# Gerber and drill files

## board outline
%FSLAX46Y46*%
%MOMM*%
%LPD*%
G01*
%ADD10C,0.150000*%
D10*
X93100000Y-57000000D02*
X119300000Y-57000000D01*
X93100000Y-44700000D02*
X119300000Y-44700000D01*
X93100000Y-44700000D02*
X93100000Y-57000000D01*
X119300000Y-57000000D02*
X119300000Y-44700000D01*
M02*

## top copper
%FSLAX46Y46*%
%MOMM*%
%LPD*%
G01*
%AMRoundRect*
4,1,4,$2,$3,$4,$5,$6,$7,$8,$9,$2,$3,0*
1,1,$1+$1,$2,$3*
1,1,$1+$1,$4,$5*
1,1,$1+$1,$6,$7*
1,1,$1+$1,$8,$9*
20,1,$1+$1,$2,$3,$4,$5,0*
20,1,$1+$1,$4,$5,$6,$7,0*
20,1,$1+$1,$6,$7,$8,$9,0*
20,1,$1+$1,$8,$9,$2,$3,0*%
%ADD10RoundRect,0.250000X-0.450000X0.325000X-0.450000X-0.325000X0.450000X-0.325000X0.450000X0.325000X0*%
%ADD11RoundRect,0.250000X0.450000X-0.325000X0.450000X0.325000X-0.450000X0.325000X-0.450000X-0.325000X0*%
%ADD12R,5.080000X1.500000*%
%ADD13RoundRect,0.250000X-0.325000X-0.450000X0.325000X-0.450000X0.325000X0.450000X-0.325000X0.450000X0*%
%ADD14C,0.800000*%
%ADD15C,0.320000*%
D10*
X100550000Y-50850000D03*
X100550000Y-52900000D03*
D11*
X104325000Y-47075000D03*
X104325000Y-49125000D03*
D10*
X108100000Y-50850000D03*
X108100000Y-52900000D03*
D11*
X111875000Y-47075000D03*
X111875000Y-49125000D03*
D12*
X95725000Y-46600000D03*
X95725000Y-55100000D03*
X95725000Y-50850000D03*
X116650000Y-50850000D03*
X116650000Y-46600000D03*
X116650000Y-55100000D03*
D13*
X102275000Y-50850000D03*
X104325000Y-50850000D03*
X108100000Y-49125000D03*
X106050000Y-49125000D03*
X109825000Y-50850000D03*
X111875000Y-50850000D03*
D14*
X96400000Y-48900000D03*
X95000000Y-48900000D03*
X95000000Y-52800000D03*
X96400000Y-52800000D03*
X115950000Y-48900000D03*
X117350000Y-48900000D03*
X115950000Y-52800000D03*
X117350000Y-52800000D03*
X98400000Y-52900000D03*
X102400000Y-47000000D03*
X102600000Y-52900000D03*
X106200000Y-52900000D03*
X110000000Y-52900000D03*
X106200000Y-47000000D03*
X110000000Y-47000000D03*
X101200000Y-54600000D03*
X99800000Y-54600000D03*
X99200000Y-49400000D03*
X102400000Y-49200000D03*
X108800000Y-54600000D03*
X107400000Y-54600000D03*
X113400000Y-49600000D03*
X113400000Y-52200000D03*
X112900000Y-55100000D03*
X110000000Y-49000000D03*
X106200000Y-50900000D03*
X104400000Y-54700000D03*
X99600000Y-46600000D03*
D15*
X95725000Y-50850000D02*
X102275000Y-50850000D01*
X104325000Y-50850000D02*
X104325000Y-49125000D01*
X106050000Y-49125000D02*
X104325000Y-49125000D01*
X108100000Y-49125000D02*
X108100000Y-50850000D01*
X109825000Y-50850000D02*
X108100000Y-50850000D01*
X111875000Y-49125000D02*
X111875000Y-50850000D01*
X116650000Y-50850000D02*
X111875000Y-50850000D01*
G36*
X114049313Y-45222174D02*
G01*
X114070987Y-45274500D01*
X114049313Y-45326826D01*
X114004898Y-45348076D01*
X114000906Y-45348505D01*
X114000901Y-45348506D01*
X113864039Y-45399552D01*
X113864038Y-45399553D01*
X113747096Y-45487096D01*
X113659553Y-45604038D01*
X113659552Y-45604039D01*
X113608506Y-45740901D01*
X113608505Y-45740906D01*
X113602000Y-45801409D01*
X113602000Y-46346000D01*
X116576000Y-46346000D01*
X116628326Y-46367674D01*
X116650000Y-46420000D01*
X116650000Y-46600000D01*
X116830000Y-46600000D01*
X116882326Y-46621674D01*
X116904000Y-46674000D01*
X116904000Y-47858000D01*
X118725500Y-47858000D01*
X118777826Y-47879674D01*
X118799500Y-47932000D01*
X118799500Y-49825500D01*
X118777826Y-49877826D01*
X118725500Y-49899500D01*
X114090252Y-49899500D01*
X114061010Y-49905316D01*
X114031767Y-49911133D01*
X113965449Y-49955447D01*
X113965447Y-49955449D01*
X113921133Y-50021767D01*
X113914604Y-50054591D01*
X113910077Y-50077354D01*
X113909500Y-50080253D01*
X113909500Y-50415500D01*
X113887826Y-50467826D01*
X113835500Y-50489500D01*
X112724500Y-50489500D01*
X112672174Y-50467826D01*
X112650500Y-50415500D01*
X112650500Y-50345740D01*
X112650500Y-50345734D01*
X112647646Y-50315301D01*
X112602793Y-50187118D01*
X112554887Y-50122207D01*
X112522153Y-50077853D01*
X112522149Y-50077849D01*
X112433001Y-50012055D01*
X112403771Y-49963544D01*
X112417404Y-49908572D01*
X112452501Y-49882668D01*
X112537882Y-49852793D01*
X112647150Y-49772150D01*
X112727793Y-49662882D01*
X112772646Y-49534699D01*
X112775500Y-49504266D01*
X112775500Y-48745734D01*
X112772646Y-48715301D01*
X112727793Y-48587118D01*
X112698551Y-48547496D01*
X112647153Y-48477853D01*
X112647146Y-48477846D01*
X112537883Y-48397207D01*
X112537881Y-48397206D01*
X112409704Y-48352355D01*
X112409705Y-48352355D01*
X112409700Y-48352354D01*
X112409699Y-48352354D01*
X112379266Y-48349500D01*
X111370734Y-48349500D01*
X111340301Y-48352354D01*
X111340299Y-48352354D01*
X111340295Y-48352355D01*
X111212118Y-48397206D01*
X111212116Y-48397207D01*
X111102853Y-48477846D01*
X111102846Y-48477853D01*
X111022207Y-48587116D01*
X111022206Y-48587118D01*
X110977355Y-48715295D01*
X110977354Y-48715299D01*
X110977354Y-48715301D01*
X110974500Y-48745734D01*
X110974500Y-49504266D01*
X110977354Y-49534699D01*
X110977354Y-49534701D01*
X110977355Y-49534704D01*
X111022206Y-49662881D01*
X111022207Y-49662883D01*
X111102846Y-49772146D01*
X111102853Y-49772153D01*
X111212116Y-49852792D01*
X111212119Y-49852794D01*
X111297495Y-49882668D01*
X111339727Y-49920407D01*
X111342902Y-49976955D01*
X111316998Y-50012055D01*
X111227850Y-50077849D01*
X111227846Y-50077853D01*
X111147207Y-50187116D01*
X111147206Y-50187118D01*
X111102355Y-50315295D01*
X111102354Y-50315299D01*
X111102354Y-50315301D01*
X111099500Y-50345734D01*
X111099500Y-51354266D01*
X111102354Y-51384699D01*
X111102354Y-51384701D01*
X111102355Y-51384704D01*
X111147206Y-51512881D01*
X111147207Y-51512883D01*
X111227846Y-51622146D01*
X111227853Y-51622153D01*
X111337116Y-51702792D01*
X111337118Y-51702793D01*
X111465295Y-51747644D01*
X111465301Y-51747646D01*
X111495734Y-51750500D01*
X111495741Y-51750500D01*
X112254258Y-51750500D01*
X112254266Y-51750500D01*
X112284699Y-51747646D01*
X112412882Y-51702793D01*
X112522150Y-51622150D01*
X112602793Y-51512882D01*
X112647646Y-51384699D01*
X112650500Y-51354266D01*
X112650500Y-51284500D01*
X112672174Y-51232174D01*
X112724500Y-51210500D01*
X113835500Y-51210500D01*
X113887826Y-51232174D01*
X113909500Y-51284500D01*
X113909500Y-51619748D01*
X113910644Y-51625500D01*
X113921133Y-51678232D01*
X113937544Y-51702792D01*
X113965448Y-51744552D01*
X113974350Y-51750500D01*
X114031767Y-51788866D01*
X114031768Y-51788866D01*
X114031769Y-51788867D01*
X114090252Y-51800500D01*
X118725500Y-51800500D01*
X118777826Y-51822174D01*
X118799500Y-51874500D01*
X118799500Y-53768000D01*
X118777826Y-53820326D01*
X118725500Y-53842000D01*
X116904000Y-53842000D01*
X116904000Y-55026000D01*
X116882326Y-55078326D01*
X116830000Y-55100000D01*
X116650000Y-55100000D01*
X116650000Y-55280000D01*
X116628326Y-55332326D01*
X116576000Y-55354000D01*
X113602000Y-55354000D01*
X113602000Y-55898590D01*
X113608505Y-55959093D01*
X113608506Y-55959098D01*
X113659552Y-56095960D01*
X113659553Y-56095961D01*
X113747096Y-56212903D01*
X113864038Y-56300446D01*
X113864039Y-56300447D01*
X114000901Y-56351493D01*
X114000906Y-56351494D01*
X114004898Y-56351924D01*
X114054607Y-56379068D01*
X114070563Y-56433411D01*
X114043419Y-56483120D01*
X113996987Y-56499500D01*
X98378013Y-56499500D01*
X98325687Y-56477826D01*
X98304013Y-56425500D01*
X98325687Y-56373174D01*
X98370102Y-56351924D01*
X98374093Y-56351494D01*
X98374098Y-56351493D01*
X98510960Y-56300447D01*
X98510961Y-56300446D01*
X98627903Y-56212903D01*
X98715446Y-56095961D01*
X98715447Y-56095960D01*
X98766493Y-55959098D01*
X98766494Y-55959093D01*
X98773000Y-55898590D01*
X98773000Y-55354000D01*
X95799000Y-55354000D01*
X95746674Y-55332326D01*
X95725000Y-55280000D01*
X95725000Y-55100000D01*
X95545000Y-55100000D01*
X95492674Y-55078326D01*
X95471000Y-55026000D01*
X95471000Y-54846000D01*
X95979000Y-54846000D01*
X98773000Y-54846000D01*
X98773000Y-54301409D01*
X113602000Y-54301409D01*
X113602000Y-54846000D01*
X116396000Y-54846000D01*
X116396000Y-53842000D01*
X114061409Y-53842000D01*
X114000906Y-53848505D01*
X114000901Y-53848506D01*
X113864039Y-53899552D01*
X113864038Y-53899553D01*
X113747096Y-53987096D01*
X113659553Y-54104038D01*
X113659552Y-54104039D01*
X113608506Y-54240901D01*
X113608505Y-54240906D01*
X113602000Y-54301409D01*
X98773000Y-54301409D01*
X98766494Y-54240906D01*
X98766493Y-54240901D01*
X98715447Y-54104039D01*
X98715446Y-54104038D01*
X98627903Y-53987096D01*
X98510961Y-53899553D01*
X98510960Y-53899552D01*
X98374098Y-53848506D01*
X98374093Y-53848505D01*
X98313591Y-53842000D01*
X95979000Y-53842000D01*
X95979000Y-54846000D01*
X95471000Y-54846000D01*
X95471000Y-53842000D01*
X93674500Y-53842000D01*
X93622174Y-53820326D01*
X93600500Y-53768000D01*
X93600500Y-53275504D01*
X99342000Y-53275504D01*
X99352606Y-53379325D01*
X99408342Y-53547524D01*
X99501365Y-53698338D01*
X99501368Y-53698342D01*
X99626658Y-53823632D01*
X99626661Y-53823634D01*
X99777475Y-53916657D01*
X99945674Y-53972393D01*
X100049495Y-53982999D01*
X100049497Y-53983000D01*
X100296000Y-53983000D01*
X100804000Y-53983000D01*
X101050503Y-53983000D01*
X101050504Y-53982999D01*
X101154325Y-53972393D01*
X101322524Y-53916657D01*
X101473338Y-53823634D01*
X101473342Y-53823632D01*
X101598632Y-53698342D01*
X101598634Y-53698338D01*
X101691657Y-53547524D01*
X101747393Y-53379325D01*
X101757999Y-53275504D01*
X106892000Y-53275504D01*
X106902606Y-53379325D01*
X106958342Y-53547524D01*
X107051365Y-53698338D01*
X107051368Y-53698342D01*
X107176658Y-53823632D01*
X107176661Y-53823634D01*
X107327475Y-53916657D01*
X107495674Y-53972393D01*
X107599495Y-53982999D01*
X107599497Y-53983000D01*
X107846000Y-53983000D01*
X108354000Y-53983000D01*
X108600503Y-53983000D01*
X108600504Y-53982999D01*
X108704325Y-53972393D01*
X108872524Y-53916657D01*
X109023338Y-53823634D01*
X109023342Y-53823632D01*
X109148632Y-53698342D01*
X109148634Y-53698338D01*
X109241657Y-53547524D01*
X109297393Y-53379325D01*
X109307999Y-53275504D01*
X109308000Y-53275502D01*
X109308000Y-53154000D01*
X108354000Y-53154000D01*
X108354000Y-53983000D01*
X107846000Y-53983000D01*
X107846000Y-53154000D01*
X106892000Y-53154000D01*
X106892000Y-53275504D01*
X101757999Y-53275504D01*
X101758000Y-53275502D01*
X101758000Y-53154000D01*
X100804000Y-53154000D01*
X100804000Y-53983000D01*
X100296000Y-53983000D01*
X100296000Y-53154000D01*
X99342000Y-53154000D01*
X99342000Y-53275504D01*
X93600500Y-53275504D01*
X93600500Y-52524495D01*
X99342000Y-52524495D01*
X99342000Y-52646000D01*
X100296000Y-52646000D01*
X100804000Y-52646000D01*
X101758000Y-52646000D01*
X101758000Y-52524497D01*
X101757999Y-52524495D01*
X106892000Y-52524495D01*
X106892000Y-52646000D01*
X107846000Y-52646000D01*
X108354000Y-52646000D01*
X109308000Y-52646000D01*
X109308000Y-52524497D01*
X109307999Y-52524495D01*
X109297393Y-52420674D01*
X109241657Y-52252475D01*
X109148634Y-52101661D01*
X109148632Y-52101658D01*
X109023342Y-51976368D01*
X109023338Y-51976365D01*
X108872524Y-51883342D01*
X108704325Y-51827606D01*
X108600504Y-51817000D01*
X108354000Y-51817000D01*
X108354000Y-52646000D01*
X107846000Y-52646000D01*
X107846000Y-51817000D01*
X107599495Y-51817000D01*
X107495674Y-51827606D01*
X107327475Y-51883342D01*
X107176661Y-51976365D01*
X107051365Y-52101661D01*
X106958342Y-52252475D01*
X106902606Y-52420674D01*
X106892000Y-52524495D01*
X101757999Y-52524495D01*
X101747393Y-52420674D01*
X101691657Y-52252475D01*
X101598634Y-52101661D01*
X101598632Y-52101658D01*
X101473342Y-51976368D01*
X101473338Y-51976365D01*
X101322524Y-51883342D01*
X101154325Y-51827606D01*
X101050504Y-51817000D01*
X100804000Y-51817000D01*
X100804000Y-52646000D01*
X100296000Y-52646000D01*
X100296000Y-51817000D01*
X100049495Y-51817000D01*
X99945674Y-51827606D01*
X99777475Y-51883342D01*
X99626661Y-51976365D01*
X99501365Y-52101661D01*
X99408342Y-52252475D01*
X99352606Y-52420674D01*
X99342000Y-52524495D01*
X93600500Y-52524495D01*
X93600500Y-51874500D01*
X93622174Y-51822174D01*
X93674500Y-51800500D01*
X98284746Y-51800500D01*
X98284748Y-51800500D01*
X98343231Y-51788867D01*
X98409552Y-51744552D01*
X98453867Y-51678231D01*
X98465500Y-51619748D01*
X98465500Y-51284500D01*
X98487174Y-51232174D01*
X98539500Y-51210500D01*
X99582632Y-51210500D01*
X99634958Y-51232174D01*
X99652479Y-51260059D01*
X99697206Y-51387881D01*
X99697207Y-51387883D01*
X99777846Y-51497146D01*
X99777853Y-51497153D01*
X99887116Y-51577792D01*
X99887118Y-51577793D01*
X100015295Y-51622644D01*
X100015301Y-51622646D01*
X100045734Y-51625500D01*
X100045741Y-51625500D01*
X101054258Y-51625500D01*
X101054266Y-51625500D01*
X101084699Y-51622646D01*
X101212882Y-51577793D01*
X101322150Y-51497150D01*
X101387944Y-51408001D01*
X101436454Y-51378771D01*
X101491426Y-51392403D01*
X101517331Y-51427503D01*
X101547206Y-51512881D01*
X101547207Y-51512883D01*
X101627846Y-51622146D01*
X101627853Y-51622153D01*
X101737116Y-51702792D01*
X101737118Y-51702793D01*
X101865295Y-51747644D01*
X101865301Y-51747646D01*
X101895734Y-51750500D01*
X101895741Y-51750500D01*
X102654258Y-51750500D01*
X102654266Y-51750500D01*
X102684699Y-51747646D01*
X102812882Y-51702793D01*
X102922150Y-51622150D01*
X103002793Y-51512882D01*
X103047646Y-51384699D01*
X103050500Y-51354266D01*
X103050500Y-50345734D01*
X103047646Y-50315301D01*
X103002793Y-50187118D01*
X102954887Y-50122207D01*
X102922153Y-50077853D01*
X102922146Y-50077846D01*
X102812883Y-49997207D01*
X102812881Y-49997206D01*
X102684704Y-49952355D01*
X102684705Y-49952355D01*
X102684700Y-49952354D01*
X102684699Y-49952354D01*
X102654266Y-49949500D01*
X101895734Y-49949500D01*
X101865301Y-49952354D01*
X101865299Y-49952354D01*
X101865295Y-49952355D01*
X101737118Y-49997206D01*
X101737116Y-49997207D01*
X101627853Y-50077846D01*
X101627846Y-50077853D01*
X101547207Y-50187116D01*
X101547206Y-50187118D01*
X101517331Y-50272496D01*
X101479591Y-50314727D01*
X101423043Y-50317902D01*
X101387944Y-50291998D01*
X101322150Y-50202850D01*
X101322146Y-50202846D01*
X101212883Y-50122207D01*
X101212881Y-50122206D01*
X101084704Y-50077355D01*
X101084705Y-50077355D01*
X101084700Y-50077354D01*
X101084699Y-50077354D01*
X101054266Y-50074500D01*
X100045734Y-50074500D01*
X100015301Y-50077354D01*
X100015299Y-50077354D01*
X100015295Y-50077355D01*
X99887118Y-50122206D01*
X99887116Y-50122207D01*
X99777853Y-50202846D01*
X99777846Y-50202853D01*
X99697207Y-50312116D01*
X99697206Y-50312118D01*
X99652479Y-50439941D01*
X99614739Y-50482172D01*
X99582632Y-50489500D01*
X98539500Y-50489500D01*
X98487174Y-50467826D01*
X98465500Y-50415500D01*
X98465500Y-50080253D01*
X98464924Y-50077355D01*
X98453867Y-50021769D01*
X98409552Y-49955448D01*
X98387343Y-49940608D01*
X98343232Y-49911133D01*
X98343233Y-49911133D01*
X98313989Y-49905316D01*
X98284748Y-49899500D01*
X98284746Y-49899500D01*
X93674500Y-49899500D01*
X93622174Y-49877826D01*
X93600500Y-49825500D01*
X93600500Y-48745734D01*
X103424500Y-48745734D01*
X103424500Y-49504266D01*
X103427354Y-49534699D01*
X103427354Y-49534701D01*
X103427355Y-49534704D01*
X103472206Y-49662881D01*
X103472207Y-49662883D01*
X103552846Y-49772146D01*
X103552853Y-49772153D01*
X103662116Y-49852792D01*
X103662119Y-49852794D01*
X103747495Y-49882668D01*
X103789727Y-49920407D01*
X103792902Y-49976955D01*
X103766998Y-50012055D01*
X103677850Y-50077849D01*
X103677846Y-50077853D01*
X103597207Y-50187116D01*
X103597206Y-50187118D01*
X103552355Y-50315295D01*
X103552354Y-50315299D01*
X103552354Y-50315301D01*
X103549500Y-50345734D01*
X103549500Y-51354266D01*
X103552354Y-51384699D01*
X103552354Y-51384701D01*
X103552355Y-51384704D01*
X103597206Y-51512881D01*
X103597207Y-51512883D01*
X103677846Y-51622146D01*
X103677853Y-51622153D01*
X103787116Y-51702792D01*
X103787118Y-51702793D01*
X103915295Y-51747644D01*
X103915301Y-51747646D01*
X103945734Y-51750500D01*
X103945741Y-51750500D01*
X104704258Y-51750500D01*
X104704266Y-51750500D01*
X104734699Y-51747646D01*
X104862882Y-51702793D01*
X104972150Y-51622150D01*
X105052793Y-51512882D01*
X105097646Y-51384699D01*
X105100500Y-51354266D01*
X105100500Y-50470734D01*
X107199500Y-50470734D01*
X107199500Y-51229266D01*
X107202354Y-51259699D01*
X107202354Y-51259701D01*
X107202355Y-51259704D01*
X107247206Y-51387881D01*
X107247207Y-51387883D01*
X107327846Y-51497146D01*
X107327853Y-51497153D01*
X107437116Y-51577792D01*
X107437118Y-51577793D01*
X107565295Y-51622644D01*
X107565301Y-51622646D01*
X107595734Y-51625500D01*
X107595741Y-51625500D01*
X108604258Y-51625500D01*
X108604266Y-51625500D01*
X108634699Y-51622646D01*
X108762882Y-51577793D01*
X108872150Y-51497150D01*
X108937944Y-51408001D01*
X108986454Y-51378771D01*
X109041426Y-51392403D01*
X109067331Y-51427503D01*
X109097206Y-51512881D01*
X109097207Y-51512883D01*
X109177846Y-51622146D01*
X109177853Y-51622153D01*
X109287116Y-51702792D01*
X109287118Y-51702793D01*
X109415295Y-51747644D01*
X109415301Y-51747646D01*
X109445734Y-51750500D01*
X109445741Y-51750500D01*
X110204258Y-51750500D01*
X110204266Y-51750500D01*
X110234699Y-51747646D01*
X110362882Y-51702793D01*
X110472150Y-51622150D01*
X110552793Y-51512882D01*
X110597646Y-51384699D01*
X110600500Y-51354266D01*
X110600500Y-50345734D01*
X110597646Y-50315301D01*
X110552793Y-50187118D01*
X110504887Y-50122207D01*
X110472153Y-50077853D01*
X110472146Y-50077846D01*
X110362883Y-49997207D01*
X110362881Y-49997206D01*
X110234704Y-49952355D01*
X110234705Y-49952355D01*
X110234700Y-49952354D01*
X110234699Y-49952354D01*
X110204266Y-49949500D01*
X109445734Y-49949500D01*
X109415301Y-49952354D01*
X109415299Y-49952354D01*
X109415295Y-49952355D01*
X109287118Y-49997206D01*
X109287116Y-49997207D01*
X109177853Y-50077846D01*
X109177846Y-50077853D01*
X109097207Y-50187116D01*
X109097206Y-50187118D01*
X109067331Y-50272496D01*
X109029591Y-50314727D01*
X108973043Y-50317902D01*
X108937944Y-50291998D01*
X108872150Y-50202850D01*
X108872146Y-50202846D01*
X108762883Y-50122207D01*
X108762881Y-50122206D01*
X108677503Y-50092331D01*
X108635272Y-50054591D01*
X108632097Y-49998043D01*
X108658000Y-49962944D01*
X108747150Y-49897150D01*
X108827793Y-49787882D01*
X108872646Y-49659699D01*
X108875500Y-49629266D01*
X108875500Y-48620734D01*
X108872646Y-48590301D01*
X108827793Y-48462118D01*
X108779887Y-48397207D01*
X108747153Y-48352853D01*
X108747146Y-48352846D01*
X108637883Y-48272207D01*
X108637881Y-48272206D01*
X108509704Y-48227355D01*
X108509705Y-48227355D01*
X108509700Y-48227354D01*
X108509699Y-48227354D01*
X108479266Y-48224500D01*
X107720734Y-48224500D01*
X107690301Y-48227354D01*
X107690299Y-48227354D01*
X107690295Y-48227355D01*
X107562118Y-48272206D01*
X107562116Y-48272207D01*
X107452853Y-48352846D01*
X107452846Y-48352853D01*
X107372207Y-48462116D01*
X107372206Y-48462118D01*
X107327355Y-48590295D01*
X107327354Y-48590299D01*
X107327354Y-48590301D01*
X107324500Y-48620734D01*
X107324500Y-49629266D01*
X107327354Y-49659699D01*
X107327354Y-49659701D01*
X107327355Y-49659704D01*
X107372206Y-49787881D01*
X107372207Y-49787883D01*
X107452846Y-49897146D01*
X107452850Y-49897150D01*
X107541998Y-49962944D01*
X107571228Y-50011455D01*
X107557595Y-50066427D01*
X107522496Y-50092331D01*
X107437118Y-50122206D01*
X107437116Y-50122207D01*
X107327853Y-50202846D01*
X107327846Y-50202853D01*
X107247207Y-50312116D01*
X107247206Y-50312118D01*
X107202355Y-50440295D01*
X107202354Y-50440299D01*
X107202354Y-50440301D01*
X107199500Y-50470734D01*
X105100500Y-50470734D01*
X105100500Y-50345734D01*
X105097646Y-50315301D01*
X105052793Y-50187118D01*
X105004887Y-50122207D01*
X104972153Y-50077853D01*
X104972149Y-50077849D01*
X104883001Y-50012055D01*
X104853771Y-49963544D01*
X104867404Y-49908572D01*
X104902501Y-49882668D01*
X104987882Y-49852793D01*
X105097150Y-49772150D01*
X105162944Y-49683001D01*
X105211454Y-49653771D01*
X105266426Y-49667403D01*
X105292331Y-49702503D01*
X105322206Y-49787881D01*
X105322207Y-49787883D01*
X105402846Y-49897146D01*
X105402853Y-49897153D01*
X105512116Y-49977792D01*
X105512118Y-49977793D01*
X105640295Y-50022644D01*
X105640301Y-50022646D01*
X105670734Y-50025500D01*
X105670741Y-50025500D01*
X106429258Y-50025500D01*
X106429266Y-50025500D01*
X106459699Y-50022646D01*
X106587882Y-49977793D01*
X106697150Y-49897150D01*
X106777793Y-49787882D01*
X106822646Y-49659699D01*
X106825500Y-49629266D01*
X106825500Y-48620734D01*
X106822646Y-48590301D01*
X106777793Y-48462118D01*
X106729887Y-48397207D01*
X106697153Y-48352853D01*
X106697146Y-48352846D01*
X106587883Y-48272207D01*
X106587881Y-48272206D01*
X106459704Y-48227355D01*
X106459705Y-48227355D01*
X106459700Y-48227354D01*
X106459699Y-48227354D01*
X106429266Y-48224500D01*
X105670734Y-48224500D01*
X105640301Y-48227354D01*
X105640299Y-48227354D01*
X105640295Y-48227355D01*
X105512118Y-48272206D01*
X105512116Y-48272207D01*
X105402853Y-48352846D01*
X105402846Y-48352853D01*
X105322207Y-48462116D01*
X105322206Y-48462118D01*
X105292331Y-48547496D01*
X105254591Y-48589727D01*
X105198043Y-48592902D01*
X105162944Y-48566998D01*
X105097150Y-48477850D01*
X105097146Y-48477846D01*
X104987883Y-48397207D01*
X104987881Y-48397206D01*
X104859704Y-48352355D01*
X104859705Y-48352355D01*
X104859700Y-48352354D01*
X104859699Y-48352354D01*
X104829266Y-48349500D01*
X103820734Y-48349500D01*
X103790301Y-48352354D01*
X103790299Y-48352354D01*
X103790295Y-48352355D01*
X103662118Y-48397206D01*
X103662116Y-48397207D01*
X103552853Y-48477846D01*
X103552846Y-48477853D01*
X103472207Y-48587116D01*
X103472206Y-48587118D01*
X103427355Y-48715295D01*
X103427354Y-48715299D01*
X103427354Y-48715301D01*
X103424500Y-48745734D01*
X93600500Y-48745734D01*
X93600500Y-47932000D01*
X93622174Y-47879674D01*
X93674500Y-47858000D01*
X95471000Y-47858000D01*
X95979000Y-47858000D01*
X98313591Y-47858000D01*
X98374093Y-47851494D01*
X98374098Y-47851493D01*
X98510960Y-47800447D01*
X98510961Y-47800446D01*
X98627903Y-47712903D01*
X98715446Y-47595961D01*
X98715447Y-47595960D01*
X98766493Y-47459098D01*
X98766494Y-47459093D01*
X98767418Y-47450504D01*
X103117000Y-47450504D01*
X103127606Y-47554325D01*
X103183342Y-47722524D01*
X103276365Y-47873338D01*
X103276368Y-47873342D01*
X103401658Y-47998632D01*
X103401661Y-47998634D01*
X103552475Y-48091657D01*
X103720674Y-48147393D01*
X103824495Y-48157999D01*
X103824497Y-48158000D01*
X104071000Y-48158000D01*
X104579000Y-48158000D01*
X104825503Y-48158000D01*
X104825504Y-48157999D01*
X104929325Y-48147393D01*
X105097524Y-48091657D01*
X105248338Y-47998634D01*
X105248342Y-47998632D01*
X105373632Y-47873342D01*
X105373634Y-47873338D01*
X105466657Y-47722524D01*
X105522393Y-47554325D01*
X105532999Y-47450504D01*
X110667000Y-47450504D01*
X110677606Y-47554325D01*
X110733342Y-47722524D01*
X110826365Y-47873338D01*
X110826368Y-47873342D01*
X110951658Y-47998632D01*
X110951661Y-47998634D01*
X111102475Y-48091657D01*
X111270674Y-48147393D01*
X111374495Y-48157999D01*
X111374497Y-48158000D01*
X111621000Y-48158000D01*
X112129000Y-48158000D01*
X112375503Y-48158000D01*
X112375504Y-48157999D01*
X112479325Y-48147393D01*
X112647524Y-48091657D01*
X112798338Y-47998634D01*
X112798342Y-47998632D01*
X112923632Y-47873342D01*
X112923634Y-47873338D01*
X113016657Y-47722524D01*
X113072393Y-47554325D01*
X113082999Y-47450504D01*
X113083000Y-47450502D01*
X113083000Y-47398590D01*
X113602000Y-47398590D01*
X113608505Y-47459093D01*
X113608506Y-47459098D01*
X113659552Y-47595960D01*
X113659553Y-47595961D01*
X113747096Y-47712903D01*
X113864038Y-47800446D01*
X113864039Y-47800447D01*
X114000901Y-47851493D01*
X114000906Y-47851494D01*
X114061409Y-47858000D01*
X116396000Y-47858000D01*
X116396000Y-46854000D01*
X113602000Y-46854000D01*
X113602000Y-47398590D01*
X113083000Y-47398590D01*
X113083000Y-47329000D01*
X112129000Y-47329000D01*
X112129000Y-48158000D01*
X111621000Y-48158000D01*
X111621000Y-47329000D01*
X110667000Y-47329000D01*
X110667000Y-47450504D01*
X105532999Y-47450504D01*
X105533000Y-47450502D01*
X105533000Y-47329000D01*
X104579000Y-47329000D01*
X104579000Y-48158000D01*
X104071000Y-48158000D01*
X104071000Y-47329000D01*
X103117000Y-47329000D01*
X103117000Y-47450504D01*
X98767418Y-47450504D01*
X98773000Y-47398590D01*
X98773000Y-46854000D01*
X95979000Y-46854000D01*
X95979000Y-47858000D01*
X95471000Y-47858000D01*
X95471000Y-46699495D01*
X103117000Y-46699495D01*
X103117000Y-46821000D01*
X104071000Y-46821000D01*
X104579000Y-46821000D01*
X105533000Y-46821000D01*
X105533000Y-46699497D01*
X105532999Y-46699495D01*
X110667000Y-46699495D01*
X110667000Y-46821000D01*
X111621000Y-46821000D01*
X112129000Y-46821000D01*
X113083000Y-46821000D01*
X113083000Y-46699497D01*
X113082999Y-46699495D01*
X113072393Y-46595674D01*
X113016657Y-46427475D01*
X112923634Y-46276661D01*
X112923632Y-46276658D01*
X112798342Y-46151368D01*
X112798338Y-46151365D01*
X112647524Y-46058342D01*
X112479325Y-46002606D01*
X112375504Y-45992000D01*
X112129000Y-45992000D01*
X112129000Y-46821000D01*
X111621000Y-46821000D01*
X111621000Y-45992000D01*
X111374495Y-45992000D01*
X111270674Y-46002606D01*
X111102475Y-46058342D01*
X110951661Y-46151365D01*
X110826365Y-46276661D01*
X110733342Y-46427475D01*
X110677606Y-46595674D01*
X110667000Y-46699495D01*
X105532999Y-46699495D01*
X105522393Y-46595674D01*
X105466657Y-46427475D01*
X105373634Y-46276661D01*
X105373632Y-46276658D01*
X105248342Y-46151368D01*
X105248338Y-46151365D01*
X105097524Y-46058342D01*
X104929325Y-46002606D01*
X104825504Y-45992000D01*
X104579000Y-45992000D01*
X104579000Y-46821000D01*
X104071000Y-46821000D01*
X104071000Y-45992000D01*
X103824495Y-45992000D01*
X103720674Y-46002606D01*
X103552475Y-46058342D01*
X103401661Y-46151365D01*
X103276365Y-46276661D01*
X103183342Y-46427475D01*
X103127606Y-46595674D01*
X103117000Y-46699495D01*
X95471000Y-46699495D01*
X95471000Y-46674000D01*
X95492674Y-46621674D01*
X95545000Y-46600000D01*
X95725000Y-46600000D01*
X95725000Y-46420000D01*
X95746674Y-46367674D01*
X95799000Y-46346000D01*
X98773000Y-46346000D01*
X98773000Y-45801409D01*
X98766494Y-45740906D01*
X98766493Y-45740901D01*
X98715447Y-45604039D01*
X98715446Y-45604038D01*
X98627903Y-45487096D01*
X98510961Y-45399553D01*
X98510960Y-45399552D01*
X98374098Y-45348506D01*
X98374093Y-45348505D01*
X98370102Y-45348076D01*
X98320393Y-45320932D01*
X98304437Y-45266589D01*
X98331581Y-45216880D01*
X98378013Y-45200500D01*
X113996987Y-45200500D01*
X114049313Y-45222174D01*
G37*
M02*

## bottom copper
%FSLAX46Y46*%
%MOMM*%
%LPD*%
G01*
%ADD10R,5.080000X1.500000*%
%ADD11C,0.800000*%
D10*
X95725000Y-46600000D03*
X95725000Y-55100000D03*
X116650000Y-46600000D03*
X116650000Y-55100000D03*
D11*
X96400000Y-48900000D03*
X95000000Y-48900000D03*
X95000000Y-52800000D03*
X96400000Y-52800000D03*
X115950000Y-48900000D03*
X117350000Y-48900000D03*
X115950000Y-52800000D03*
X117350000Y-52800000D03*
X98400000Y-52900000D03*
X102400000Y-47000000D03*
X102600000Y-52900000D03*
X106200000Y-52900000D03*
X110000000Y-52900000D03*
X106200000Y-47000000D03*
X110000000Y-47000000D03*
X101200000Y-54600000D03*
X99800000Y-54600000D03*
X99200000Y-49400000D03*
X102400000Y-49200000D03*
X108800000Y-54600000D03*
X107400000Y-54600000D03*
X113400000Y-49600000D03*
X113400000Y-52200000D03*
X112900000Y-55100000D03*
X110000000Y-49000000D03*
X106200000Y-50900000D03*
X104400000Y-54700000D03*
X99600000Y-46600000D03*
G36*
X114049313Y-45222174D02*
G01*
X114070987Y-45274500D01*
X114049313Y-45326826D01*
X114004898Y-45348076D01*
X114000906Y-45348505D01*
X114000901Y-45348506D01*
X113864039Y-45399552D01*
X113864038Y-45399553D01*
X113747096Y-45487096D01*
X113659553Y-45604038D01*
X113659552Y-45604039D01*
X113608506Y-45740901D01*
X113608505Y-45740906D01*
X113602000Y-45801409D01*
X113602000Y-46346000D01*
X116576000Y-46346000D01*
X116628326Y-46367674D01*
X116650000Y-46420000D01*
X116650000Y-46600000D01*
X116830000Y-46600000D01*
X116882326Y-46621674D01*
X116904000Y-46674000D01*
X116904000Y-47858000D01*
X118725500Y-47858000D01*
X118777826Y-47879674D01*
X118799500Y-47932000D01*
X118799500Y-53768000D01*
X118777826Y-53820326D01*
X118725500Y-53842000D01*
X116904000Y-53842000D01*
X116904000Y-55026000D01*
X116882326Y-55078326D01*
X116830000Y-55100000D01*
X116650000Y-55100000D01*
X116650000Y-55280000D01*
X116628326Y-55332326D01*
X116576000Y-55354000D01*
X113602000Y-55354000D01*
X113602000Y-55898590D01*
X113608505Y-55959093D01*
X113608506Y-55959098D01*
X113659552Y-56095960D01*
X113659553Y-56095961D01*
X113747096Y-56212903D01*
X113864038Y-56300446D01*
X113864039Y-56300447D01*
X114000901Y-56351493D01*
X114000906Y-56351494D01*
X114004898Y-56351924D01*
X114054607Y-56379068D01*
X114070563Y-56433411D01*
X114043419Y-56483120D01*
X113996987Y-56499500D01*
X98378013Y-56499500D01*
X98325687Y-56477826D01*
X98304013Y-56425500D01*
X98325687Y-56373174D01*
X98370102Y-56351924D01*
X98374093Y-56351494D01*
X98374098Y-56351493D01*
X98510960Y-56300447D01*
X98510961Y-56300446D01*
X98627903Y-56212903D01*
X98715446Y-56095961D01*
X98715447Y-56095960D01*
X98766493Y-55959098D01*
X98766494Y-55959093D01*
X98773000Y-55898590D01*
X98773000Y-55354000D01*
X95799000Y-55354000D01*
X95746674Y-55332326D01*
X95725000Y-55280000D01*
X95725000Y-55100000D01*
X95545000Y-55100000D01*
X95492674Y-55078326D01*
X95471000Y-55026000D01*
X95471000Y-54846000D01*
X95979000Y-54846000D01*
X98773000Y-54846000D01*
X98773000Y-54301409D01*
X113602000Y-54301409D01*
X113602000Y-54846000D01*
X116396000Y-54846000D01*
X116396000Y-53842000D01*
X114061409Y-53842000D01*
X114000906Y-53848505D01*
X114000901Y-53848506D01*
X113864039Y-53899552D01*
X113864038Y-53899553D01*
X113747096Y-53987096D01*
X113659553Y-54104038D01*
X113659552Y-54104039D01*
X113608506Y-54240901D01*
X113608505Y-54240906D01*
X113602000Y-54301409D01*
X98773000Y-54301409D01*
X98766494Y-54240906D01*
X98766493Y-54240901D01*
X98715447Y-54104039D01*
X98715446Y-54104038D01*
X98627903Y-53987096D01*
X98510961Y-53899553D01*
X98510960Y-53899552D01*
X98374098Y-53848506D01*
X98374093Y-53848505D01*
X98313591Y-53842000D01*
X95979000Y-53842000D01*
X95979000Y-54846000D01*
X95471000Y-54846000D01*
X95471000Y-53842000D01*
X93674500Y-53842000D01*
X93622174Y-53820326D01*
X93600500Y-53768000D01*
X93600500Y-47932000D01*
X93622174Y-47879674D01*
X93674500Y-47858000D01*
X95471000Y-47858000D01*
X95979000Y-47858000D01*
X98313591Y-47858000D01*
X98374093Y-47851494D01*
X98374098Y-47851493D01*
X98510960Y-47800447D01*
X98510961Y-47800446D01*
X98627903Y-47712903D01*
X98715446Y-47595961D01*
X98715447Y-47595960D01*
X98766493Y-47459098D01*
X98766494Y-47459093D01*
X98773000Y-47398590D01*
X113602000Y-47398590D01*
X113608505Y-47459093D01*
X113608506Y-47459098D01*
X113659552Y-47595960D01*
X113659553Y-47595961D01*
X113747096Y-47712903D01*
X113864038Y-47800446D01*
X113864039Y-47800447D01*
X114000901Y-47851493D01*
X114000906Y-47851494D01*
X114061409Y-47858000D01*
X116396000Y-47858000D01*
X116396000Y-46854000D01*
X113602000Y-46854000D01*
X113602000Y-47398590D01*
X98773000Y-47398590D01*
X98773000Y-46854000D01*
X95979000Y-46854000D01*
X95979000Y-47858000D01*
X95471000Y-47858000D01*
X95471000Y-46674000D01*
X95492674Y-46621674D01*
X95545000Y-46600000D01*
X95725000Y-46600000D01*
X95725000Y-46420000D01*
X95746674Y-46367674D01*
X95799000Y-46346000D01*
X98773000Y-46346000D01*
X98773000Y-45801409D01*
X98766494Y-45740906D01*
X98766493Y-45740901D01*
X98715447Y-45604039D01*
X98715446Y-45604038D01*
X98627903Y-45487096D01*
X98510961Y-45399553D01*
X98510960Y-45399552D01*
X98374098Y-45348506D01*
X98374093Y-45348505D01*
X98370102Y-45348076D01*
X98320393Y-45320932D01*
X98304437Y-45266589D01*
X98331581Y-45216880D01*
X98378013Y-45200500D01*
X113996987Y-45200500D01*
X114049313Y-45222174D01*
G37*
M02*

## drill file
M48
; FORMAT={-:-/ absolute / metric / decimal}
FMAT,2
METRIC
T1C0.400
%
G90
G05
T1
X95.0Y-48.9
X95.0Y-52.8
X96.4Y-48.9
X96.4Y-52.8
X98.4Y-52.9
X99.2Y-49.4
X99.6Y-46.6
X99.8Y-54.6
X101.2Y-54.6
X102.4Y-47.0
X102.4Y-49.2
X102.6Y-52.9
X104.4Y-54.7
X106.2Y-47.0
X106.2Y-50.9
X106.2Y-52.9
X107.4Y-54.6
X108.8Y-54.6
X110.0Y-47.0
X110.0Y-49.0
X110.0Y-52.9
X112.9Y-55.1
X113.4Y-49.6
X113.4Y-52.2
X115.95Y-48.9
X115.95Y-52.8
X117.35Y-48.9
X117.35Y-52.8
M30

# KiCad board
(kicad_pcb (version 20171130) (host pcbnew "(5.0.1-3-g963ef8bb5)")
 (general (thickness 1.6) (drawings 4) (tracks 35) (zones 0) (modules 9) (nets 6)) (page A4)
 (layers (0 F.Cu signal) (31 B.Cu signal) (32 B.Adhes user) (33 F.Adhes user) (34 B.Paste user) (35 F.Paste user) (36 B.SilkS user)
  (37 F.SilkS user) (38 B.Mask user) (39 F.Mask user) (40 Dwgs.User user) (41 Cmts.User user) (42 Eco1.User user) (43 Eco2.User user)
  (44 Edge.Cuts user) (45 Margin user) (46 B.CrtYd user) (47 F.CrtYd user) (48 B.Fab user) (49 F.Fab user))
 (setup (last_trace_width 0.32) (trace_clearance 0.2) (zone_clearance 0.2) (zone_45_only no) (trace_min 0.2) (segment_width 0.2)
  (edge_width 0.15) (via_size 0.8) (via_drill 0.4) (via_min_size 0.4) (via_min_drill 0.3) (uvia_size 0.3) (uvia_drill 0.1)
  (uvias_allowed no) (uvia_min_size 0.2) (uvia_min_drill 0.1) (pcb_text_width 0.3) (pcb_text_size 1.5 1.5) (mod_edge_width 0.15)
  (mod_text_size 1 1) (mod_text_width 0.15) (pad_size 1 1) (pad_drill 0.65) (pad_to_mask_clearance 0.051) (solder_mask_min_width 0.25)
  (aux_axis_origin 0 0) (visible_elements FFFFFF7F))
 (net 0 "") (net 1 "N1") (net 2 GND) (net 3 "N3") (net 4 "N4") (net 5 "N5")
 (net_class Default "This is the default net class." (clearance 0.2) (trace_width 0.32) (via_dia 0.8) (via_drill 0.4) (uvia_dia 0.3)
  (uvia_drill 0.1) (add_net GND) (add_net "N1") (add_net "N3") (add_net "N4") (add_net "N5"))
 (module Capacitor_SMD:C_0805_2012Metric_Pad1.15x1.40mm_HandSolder (layer F.Cu) (at 100.55 51.875 270)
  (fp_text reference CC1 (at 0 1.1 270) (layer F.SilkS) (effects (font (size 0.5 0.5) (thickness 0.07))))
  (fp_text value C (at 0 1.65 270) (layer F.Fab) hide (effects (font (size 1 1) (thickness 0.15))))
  (pad 1 smd roundrect (at -1.025 0 270) (size 1.15 1.4) (layers F.Cu F.Paste F.Mask) (roundrect_rratio 0.217391) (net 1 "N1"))
  (pad 2 smd roundrect (at 1.025 0 270) (size 1.15 1.4) (layers F.Cu F.Paste F.Mask) (roundrect_rratio 0.217391) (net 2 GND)))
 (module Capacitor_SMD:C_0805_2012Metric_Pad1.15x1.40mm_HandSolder (layer F.Cu) (at 104.325 48.1 90)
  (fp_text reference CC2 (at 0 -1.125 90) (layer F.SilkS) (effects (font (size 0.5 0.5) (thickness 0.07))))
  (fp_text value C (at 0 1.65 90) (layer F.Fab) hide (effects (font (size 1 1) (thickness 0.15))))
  (pad 2 smd roundrect (at 1.025 0 90) (size 1.15 1.4) (layers F.Cu F.Paste F.Mask) (roundrect_rratio 0.217391) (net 2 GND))
  (pad 1 smd roundrect (at -1.025 0 90) (size 1.15 1.4) (layers F.Cu F.Paste F.Mask) (roundrect_rratio 0.217391) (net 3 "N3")))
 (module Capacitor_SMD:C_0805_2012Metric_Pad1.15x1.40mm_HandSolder (layer F.Cu) (at 108.1 51.875 270)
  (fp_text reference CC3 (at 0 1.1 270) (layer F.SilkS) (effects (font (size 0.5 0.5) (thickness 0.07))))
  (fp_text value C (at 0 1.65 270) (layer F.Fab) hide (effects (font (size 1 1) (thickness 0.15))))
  (pad 1 smd roundrect (at -1.025 0 270) (size 1.15 1.4) (layers F.Cu F.Paste F.Mask) (roundrect_rratio 0.217391) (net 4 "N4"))
  (pad 2 smd roundrect (at 1.025 0 270) (size 1.15 1.4) (layers F.Cu F.Paste F.Mask) (roundrect_rratio 0.217391) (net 2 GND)))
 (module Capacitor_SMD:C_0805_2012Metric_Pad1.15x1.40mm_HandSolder (layer F.Cu) (at 111.875 48.1 90)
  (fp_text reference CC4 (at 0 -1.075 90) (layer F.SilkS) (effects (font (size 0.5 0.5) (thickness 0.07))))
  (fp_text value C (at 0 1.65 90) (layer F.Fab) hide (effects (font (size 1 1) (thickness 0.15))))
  (pad 2 smd roundrect (at 1.025 0 90) (size 1.15 1.4) (layers F.Cu F.Paste F.Mask) (roundrect_rratio 0.217391) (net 2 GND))
  (pad 1 smd roundrect (at -1.025 0 90) (size 1.15 1.4) (layers F.Cu F.Paste F.Mask) (roundrect_rratio 0.217391) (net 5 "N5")))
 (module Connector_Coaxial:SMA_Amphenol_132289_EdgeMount (layer F.Cu) (at 95.725 50.85 180)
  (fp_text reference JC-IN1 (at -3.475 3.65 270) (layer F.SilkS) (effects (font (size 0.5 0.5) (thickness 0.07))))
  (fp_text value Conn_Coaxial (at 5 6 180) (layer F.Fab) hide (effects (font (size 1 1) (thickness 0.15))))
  (pad 2 smd rect (at 0 4.25 270) (size 1.5 5.08) (layers B.Cu B.Paste B.Mask) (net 2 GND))
  (pad 2 smd rect (at 0 -4.25 270) (size 1.5 5.08) (layers B.Cu B.Paste B.Mask) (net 2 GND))
  (pad 2 smd rect (at 0 4.25 270) (size 1.5 5.08) (layers F.Cu F.Paste F.Mask) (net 2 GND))
  (pad 2 smd rect (at 0 -4.25 270) (size 1.5 5.08) (layers F.Cu F.Paste F.Mask) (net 2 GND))
  (pad 1 smd rect (at 0 0 270) (size 1.5 5.08) (layers F.Cu F.Paste F.Mask) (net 1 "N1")))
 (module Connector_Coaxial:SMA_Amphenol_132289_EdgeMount (layer F.Cu) (at 116.65 50.85)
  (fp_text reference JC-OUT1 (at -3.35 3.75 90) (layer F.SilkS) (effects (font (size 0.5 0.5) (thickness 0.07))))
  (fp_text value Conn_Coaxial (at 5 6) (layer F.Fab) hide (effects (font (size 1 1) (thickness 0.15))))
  (pad 1 smd rect (at 0 0 90) (size 1.5 5.08) (layers F.Cu F.Paste F.Mask) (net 5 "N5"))
  (pad 2 smd rect (at 0 -4.25 90) (size 1.5 5.08) (layers F.Cu F.Paste F.Mask) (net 2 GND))
  (pad 2 smd rect (at 0 4.25 90) (size 1.5 5.08) (layers F.Cu F.Paste F.Mask) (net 2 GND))
  (pad 2 smd rect (at 0 -4.25 90) (size 1.5 5.08) (layers B.Cu B.Paste B.Mask) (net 2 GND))
  (pad 2 smd rect (at 0 4.25 90) (size 1.5 5.08) (layers B.Cu B.Paste B.Mask) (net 2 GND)))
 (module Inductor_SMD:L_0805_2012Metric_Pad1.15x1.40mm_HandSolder (layer F.Cu) (at 103.3 50.85)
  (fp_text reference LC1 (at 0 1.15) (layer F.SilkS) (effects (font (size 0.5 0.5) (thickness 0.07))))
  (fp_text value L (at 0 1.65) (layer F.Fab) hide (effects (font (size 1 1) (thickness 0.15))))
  (pad 1 smd roundrect (at -1.025 0) (size 1.15 1.4) (layers F.Cu F.Paste F.Mask) (roundrect_rratio 0.217391) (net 1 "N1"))
  (pad 2 smd roundrect (at 1.025 0) (size 1.15 1.4) (layers F.Cu F.Paste F.Mask) (roundrect_rratio 0.217391) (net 3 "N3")))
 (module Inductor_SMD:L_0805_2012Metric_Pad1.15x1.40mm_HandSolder (layer F.Cu) (at 107.075 49.125)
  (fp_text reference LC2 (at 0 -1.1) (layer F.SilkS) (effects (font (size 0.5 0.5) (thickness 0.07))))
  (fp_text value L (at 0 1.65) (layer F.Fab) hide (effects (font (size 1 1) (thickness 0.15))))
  (pad 2 smd roundrect (at 1.025 0) (size 1.15 1.4) (layers F.Cu F.Paste F.Mask) (roundrect_rratio 0.217391) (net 4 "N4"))
  (pad 1 smd roundrect (at -1.025 0) (size 1.15 1.4) (layers F.Cu F.Paste F.Mask) (roundrect_rratio 0.217391) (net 3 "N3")))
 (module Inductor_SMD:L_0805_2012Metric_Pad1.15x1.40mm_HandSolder (layer F.Cu) (at 110.85 50.85)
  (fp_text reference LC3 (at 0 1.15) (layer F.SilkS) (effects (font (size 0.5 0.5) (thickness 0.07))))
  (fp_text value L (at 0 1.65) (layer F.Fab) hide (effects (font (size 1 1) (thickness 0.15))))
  (pad 1 smd roundrect (at -1.025 0) (size 1.15 1.4) (layers F.Cu F.Paste F.Mask) (roundrect_rratio 0.217391) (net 4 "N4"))
  (pad 2 smd roundrect (at 1.025 0) (size 1.15 1.4) (layers F.Cu F.Paste F.Mask) (roundrect_rratio 0.217391) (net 5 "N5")))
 (gr_line (start 93.1 57) (end 119.3 57) (layer Edge.Cuts) (width 0.15))
 (gr_line (start 93.1 44.7) (end 119.3 44.7) (layer Edge.Cuts) (width 0.15))
 (gr_line (start 93.1 44.7) (end 93.1 57) (layer Edge.Cuts) (width 0.15))
 (gr_line (start 119.3 57) (end 119.3 44.7) (layer Edge.Cuts) (width 0.15))
 (via (at 96.4 48.9) (size 0.8) (drill 0.4) (layers F.Cu B.Cu) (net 2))
 (via (at 95 48.9) (size 0.8) (drill 0.4) (layers F.Cu B.Cu) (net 2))
 (via (at 95 52.8) (size 0.8) (drill 0.4) (layers F.Cu B.Cu) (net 2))
 (via (at 96.4 52.8) (size 0.8) (drill 0.4) (layers F.Cu B.Cu) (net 2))
 (via (at 115.95 48.9) (size 0.8) (drill 0.4) (layers F.Cu B.Cu) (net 2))
 (via (at 117.35 48.9) (size 0.8) (drill 0.4) (layers F.Cu B.Cu) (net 2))
 (via (at 115.95 52.8) (size 0.8) (drill 0.4) (layers F.Cu B.Cu) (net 2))
 (via (at 117.35 52.8) (size 0.8) (drill 0.4) (layers F.Cu B.Cu) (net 2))
 (via (at 98.4 52.9) (size 0.8) (drill 0.4) (layers F.Cu B.Cu) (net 2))
 (via (at 102.4 47) (size 0.8) (drill 0.4) (layers F.Cu B.Cu) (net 2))
 (via (at 102.6 52.9) (size 0.8) (drill 0.4) (layers F.Cu B.Cu) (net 2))
 (via (at 106.2 52.9) (size 0.8) (drill 0.4) (layers F.Cu B.Cu) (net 2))
 (via (at 110 52.9) (size 0.8) (drill 0.4) (layers F.Cu B.Cu) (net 2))
 (via (at 106.2 47) (size 0.8) (drill 0.4) (layers F.Cu B.Cu) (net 2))
 (via (at 110 47) (size 0.8) (drill 0.4) (layers F.Cu B.Cu) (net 2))
 (via (at 101.2 54.6) (size 0.8) (drill 0.4) (layers F.Cu B.Cu) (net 2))
 (via (at 99.8 54.6) (size 0.8) (drill 0.4) (layers F.Cu B.Cu) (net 2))
 (via (at 99.2 49.4) (size 0.8) (drill 0.4) (layers F.Cu B.Cu) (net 2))
 (via (at 102.4 49.2) (size 0.8) (drill 0.4) (layers F.Cu B.Cu) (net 2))
 (via (at 108.8 54.6) (size 0.8) (drill 0.4) (layers F.Cu B.Cu) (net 2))
 (via (at 107.4 54.6) (size 0.8) (drill 0.4) (layers F.Cu B.Cu) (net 2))
 (via (at 113.4 49.6) (size 0.8) (drill 0.4) (layers F.Cu B.Cu) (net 2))
 (via (at 113.4 52.2) (size 0.8) (drill 0.4) (layers F.Cu B.Cu) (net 2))
 (via (at 112.9 55.1) (size 0.8) (drill 0.4) (layers F.Cu B.Cu) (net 2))
 (via (at 110 49) (size 0.8) (drill 0.4) (layers F.Cu B.Cu) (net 2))
 (via (at 106.2 50.9) (size 0.8) (drill 0.4) (layers F.Cu B.Cu) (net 2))
 (via (at 104.4 54.7) (size 0.8) (drill 0.4) (layers F.Cu B.Cu) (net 2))
 (via (at 99.6 46.6) (size 0.8) (drill 0.4) (layers F.Cu B.Cu) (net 2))
 (segment (start 95.725 50.85) (end 102.275 50.85) (width 0.32) (layer F.Cu) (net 1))
 (segment (start 104.325 50.85) (end 104.325 49.125) (width 0.32) (layer F.Cu) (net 3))
 (segment (start 106.05 49.125) (end 104.325 49.125) (width 0.32) (layer F.Cu) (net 3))
 (segment (start 108.1 49.125) (end 108.1 50.85) (width 0.32) (layer F.Cu) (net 4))
 (segment (start 109.825 50.85) (end 108.1 50.85) (width 0.32) (layer F.Cu) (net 4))
 (segment (start 111.875 49.125) (end 111.875 50.85) (width 0.32) (layer F.Cu) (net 5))
 (segment (start 116.65 50.85) (end 111.875 50.85) (width 0.32) (layer F.Cu) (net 5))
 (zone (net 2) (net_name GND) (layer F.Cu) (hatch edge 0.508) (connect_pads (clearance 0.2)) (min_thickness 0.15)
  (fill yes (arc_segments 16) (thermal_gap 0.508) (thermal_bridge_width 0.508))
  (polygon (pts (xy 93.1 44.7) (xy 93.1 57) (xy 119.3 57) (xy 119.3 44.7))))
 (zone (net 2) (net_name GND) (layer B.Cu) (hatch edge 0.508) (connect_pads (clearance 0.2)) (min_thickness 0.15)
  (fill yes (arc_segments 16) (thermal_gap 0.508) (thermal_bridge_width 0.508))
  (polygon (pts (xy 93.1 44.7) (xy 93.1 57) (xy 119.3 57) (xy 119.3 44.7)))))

